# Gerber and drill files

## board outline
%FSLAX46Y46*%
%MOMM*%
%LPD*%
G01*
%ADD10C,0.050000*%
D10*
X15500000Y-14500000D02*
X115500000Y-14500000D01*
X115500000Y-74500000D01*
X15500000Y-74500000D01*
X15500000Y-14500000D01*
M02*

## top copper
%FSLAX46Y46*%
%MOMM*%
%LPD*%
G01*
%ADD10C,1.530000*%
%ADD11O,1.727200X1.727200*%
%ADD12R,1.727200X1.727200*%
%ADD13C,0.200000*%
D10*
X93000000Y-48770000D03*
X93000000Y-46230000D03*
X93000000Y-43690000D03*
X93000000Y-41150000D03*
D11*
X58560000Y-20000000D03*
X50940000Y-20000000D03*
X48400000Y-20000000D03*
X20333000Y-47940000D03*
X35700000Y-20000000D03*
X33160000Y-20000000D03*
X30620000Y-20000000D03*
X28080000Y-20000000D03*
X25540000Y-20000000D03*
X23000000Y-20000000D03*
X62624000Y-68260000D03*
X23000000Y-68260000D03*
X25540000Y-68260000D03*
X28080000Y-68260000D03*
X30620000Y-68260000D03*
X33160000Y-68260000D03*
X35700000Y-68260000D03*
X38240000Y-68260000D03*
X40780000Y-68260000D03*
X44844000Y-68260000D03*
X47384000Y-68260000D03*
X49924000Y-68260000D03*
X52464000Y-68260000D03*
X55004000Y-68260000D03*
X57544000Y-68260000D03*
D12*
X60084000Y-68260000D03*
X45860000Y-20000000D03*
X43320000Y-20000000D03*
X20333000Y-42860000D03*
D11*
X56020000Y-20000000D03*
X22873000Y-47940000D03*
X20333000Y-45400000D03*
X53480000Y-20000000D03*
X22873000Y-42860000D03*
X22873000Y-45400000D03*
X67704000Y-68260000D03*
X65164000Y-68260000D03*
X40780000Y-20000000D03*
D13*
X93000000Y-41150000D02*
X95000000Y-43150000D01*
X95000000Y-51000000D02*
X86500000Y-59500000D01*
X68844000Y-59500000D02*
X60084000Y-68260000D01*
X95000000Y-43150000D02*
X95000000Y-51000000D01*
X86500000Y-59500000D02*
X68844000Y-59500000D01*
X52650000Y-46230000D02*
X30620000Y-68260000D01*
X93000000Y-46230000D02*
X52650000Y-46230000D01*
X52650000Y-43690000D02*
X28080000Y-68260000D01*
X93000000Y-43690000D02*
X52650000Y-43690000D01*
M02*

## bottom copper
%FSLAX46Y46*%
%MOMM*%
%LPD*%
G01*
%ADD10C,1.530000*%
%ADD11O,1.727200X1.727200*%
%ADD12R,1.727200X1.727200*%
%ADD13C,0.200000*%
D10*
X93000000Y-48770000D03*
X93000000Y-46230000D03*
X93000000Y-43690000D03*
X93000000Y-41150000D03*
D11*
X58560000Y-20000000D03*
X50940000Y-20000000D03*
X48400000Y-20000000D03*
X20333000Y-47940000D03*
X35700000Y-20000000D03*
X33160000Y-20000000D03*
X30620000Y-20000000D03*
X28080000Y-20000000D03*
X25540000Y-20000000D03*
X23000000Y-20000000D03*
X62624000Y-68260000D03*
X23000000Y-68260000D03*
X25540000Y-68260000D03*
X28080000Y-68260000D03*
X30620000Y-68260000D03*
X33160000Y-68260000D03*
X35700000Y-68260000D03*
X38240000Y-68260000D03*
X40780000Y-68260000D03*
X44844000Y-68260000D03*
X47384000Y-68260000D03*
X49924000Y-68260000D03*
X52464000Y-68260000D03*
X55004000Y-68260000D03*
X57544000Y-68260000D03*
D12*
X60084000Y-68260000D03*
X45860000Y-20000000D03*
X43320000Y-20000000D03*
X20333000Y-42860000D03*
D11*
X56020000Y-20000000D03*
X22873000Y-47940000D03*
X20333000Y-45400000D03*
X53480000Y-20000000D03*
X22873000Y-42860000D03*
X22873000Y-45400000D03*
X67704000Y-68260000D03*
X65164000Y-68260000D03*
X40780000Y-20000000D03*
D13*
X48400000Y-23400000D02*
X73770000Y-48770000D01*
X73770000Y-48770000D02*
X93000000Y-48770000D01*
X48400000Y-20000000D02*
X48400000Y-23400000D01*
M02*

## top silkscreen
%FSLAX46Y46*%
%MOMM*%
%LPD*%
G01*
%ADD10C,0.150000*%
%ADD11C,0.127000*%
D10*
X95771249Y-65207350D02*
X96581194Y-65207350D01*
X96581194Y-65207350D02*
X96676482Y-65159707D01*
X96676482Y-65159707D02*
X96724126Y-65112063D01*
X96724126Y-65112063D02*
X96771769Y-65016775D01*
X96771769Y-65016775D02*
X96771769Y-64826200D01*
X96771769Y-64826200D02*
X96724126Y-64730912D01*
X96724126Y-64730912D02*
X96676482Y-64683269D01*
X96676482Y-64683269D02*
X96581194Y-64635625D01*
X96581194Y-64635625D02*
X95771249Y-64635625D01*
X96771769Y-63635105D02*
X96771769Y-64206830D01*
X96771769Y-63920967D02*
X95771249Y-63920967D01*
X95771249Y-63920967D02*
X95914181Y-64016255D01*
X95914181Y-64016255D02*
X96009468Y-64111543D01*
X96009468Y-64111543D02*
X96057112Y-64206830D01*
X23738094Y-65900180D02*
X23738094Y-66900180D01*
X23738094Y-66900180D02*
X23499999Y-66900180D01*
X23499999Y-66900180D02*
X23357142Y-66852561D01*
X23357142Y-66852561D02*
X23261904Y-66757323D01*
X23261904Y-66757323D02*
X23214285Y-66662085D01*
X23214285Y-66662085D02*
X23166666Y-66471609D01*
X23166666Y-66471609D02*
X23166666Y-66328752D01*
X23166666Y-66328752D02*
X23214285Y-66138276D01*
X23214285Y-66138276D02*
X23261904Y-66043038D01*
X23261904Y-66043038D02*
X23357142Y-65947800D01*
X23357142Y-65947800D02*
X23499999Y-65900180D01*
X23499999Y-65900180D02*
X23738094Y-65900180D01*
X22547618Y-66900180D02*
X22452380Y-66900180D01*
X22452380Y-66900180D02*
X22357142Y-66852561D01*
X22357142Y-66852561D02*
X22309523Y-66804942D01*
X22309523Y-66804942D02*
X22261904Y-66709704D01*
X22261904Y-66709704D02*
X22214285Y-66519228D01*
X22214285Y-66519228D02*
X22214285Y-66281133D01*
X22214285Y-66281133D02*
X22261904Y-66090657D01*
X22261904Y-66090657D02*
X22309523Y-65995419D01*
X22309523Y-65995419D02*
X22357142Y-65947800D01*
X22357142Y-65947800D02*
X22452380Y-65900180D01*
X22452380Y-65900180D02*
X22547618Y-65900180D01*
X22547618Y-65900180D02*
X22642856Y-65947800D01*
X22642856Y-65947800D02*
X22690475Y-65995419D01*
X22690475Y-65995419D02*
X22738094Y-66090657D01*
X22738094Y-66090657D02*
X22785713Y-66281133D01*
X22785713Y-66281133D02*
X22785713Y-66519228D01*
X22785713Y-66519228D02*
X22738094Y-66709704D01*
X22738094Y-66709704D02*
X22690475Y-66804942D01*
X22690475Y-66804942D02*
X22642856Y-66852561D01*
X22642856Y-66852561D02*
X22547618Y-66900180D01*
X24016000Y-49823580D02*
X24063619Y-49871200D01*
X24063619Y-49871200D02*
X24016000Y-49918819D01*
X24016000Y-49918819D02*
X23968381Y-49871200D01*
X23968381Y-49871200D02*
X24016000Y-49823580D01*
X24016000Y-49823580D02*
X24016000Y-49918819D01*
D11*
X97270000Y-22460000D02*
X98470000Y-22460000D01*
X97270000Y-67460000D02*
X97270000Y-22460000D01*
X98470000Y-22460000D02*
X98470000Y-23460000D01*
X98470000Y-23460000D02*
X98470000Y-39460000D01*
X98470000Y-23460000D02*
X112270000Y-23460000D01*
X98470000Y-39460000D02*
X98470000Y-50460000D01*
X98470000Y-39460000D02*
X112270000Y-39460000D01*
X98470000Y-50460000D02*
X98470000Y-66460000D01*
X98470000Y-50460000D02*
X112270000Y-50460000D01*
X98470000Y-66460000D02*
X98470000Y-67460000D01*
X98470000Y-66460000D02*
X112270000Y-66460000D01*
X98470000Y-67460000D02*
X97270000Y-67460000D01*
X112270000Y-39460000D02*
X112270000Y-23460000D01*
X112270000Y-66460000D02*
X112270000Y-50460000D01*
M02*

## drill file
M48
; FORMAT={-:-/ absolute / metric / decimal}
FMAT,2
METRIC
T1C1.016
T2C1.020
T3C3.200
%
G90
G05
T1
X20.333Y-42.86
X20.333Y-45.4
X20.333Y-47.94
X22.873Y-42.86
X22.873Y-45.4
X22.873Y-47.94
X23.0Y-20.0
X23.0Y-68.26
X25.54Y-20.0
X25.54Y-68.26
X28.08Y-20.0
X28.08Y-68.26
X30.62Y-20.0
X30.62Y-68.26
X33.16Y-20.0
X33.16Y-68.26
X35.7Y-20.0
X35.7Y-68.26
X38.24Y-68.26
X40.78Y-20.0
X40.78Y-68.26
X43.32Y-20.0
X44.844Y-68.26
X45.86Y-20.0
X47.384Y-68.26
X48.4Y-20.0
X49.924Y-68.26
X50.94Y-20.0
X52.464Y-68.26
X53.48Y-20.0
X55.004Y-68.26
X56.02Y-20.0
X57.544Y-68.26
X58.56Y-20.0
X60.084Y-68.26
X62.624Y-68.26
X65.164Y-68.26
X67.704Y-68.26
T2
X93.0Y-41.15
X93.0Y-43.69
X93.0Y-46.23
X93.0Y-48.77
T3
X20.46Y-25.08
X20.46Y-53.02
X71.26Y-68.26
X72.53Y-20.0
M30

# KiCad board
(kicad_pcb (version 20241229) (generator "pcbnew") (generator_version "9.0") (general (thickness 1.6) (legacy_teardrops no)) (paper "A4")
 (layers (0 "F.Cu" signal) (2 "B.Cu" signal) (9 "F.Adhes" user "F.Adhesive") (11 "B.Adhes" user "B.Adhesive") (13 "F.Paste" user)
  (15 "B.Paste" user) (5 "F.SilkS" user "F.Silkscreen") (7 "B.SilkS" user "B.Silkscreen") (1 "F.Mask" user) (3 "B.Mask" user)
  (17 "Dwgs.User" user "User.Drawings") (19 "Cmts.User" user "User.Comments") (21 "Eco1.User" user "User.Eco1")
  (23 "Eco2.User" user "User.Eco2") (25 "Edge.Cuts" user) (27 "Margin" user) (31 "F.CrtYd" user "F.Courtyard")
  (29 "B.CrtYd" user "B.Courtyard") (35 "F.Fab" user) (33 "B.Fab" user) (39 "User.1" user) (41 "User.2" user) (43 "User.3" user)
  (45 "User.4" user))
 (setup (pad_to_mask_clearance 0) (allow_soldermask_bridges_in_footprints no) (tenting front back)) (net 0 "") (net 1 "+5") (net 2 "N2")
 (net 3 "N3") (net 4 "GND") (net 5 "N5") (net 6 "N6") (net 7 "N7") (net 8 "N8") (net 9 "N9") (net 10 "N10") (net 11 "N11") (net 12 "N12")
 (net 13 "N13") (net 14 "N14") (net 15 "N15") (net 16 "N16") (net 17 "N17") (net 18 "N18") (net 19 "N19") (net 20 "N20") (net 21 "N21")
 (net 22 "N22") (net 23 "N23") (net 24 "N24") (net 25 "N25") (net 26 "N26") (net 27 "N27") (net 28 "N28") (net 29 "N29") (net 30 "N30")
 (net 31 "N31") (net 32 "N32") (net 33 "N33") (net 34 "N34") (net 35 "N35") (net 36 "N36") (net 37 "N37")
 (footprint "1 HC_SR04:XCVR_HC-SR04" (layer "F.Cu") (at 93 44.96 90)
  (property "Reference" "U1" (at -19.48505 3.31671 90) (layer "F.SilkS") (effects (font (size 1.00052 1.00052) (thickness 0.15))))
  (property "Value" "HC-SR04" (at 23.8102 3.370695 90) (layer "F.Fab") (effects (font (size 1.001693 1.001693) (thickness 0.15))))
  (fp_line (start 22.5 4.27) (end 22.5 5.47) (stroke (width 0.127) (type solid)) (layer "F.SilkS"))
  (fp_line (start -22.5 4.27) (end 22.5 4.27) (stroke (width 0.127) (type solid)) (layer "F.SilkS"))
  (fp_line (start 22.5 5.47) (end 21.5 5.47) (stroke (width 0.127) (type solid)) (layer "F.SilkS"))
  (fp_line (start 21.5 5.47) (end 5.5 5.47) (stroke (width 0.127) (type solid)) (layer "F.SilkS"))
  (fp_line (start 21.5 5.47) (end 21.5 19.27) (stroke (width 0.127) (type solid)) (layer "F.SilkS"))
  (fp_line (start 5.5 5.47) (end -5.5 5.47) (stroke (width 0.127) (type solid)) (layer "F.SilkS"))
  (fp_line (start 5.5 5.47) (end 5.5 19.27) (stroke (width 0.127) (type solid)) (layer "F.SilkS"))
  (fp_line (start -5.5 5.47) (end -21.5 5.47) (stroke (width 0.127) (type solid)) (layer "F.SilkS"))
  (fp_line (start -5.5 5.47) (end -5.5 19.27) (stroke (width 0.127) (type solid)) (layer "F.SilkS"))
  (fp_line (start -21.5 5.47) (end -22.5 5.47) (stroke (width 0.127) (type solid)) (layer "F.SilkS"))
  (fp_line (start -21.5 5.47) (end -21.5 19.27) (stroke (width 0.127) (type solid)) (layer "F.SilkS"))
  (fp_line (start -22.5 5.47) (end -22.5 4.27) (stroke (width 0.127) (type solid)) (layer "F.SilkS"))
  (fp_line (start 5.5 19.27) (end 21.5 19.27) (stroke (width 0.127) (type solid)) (layer "F.SilkS"))
  (fp_line (start -21.5 19.27) (end -5.5 19.27) (stroke (width 0.127) (type solid)) (layer "F.SilkS"))
  (pad "1" thru_hole circle (at -3.81 0 90) (size 1.53 1.53) (drill 1.02) (layers "*.Cu" "*.Mask") (remove_unused_layers no) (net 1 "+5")
   (solder_mask_margin 0.102))
  (pad "2" thru_hole circle (at -1.27 0 90) (size 1.53 1.53) (drill 1.02) (layers "*.Cu" "*.Mask") (remove_unused_layers no) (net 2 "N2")
   (solder_mask_margin 0.102))
  (pad "3" thru_hole circle (at 1.27 0 90) (size 1.53 1.53) (drill 1.02) (layers "*.Cu" "*.Mask") (remove_unused_layers no) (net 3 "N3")
   (solder_mask_margin 0.102))
  (pad "4" thru_hole circle (at 3.81 0 90) (size 1.53 1.53) (drill 1.02) (layers "*.Cu" "*.Mask") (remove_unused_layers no) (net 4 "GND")
   (solder_mask_margin 0.102)))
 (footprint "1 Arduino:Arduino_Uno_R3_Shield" (layer "F.Cu") (at 86.5 17.46 180)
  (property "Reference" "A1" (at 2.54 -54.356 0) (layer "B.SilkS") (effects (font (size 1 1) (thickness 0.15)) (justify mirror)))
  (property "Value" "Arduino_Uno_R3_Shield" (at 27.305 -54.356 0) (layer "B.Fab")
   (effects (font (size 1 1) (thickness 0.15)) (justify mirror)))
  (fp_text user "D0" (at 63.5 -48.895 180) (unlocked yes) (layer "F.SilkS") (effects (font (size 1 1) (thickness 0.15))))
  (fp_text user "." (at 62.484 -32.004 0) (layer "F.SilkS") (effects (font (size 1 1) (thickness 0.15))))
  (pad "" np_thru_hole circle (at 13.97 -2.54 180) (size 3.2 3.2) (drill 3.2) (layers "*.Cu" "*.Mask"))
  (pad "" np_thru_hole circle (at 15.24 -50.8 180) (size 3.2 3.2) (drill 3.2) (layers "*.Cu" "*.Mask"))
  (pad "" thru_hole oval (at 27.94 -2.54 180) (size 1.7272 1.7272) (drill 1.016) (layers "*.Cu" "*.Mask") (remove_unused_layers no))
  (pad "" np_thru_hole circle (at 66.04 -35.56 180) (size 3.2 3.2) (drill 3.2) (layers "*.Cu" "*.Mask"))
  (pad "" np_thru_hole circle (at 66.04 -7.62 180) (size 3.2 3.2) (drill 3.2) (layers "*.Cu" "*.Mask"))
  (pad "3V3" thru_hole oval (at 35.56 -2.54 180) (size 1.7272 1.7272) (drill 1.016) (layers "*.Cu" "*.Mask") (remove_unused_layers no)
   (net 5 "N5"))
  (pad "5V1" thru_hole oval (at 38.1 -2.54 180) (size 1.7272 1.7272) (drill 1.016) (layers "*.Cu" "*.Mask") (remove_unused_layers no)
   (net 1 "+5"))
  (pad "5V2" thru_hole oval (at 66.167 -30.48 180) (size 1.7272 1.7272) (drill 1.016) (layers "*.Cu" "*.Mask") (remove_unused_layers no)
   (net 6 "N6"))
  (pad "A0" thru_hole oval (at 50.8 -2.54 180) (size 1.7272 1.7272) (drill 1.016) (layers "*.Cu" "*.Mask") (remove_unused_layers no)
   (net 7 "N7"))
  (pad "A1" thru_hole oval (at 53.34 -2.54 180) (size 1.7272 1.7272) (drill 1.016) (layers "*.Cu" "*.Mask") (remove_unused_layers no)
   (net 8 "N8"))
  (pad "A2" thru_hole oval (at 55.88 -2.54 180) (size 1.7272 1.7272) (drill 1.016) (layers "*.Cu" "*.Mask") (remove_unused_layers no)
   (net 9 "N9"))
  (pad "A3" thru_hole oval (at 58.42 -2.54 180) (size 1.7272 1.7272) (drill 1.016) (layers "*.Cu" "*.Mask") (remove_unused_layers no)
   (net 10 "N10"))
  (pad "A4" thru_hole oval (at 60.96 -2.54 180) (size 1.7272 1.7272) (drill 1.016) (layers "*.Cu" "*.Mask") (remove_unused_layers no)
   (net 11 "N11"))
  (pad "A5" thru_hole oval (at 63.5 -2.54 180) (size 1.7272 1.7272) (drill 1.016) (layers "*.Cu" "*.Mask") (remove_unused_layers no)
   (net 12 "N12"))
  (pad "AREF" thru_hole oval (at 23.876 -50.8 180) (size 1.7272 1.7272) (drill 1.016) (layers "*.Cu" "*.Mask") (remove_unused_layers no)
   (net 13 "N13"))
  (pad "D0" thru_hole oval (at 63.5 -50.8 180) (size 1.7272 1.7272) (drill 1.016) (layers "*.Cu" "*.Mask") (remove_unused_layers no)
   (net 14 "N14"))
  (pad "D1" thru_hole oval (at 60.96 -50.8 180) (size 1.7272 1.7272) (drill 1.016) (layers "*.Cu" "*.Mask") (remove_unused_layers no)
   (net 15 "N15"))
  (pad "D2" thru_hole oval (at 58.42 -50.8 180) (size 1.7272 1.7272) (drill 1.016) (layers "*.Cu" "*.Mask") (remove_unused_layers no)
   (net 3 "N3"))
  (pad "D3" thru_hole oval (at 55.88 -50.8 180) (size 1.7272 1.7272) (drill 1.016) (layers "*.Cu" "*.Mask") (remove_unused_layers no)
   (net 2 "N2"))
  (pad "D4" thru_hole oval (at 53.34 -50.8 180) (size 1.7272 1.7272) (drill 1.016) (layers "*.Cu" "*.Mask") (remove_unused_layers no)
   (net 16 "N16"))
  (pad "D5" thru_hole oval (at 50.8 -50.8 180) (size 1.7272 1.7272) (drill 1.016) (layers "*.Cu" "*.Mask") (remove_unused_layers no)
   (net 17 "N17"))
  (pad "D6" thru_hole oval (at 48.26 -50.8 180) (size 1.7272 1.7272) (drill 1.016) (layers "*.Cu" "*.Mask") (remove_unused_layers no)
   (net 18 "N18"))
  (pad "D7" thru_hole oval (at 45.72 -50.8 180) (size 1.7272 1.7272) (drill 1.016) (layers "*.Cu" "*.Mask") (remove_unused_layers no)
   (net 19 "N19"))
  (pad "D8" thru_hole oval (at 41.656 -50.8 180) (size 1.7272 1.7272) (drill 1.016) (layers "*.Cu" "*.Mask") (remove_unused_layers no)
   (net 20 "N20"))
  (pad "D9" thru_hole oval (at 39.116 -50.8 180) (size 1.7272 1.7272) (drill 1.016) (layers "*.Cu" "*.Mask") (remove_unused_layers no)
   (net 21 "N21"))
  (pad "D10" thru_hole oval (at 36.576 -50.8 180) (size 1.7272 1.7272) (drill 1.016) (layers "*.Cu" "*.Mask") (remove_unused_layers no)
   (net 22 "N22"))
  (pad "D11" thru_hole oval (at 34.036 -50.8 180) (size 1.7272 1.7272) (drill 1.016) (layers "*.Cu" "*.Mask") (remove_unused_layers no)
   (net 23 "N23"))
  (pad "D12" thru_hole oval (at 31.496 -50.8 180) (size 1.7272 1.7272) (drill 1.016) (layers "*.Cu" "*.Mask") (remove_unused_layers no)
   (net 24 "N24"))
  (pad "D13" thru_hole oval (at 28.956 -50.8 180) (size 1.7272 1.7272) (drill 1.016) (layers "*.Cu" "*.Mask") (remove_unused_layers no)
   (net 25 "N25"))
  (pad "GND1" thru_hole rect (at 26.416 -50.8 180) (size 1.7272 1.7272) (drill 1.016) (layers "*.Cu" "*.Mask") (remove_unused_layers no)
   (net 4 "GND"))
  (pad "GND2" thru_hole rect (at 40.64 -2.54 180) (size 1.7272 1.7272) (drill 1.016) (layers "*.Cu" "*.Mask") (remove_unused_layers no)
   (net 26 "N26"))
  (pad "GND3" thru_hole rect (at 43.18 -2.54 180) (size 1.7272 1.7272) (drill 1.016) (layers "*.Cu" "*.Mask") (remove_unused_layers no)
   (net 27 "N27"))
  (pad "GND4" thru_hole rect (at 66.167 -25.4 180) (size 1.7272 1.7272) (drill 1.016) (layers "*.Cu" "*.Mask") (remove_unused_layers no)
   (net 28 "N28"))
  (pad "IORF" thru_hole oval (at 30.48 -2.54 180) (size 1.7272 1.7272) (drill 1.016) (layers "*.Cu" "*.Mask") (remove_unused_layers no)
   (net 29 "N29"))
  (pad "MISO" thru_hole oval (at 63.627 -30.48 180) (size 1.7272 1.7272) (drill 1.016) (layers "*.Cu" "*.Mask") (remove_unused_layers no)
   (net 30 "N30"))
  (pad "MOSI" thru_hole oval (at 66.167 -27.94 180) (size 1.7272 1.7272) (drill 1.016) (layers "*.Cu" "*.Mask") (remove_unused_layers no)
   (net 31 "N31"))
  (pad "RST1" thru_hole oval (at 33.02 -2.54 180) (size 1.7272 1.7272) (drill 1.016) (layers "*.Cu" "*.Mask") (remove_unused_layers no)
   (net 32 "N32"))
  (pad "RST2" thru_hole oval (at 63.627 -25.4 180) (size 1.7272 1.7272) (drill 1.016) (layers "*.Cu" "*.Mask") (remove_unused_layers no)
   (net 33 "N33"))
  (pad "SCK" thru_hole oval (at 63.627 -27.94 180) (size 1.7272 1.7272) (drill 1.016) (layers "*.Cu" "*.Mask") (remove_unused_layers no)
   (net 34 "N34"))
  (pad "SCL" thru_hole oval (at 18.796 -50.8 180) (size 1.7272 1.7272) (drill 1.016) (layers "*.Cu" "*.Mask") (remove_unused_layers no)
   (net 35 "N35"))
  (pad "SDA" thru_hole oval (at 21.336 -50.8 180) (size 1.7272 1.7272) (drill 1.016) (layers "*.Cu" "*.Mask") (remove_unused_layers no)
   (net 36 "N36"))
  (pad "VIN" thru_hole oval (at 45.72 -2.54 180) (size 1.7272 1.7272) (drill 1.016) (layers "*.Cu" "*.Mask") (remove_unused_layers no)
   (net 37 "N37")))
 (gr_rect (start 15.5 14.5) (end 115.5 74.5) (stroke (width 0.05) (type default)) (fill no) (layer "Edge.Cuts"))
 (segment (start 93 41.15) (end 95 43.15) (width 0.2) (layer "F.Cu") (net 4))
 (segment (start 95 51) (end 86.5 59.5) (width 0.2) (layer "F.Cu") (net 4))
 (segment (start 68.844 59.5) (end 60.084 68.26) (width 0.2) (layer "F.Cu") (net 4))
 (segment (start 95 43.15) (end 95 51) (width 0.2) (layer "F.Cu") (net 4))
 (segment (start 86.5 59.5) (end 68.844 59.5) (width 0.2) (layer "F.Cu") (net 4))
 (segment (start 52.65 46.23) (end 30.62 68.26) (width 0.2) (layer "F.Cu") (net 2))
 (segment (start 93 46.23) (end 52.65 46.23) (width 0.2) (layer "F.Cu") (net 2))
 (segment (start 52.65 43.69) (end 28.08 68.26) (width 0.2) (layer "F.Cu") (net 3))
 (segment (start 93 43.69) (end 52.65 43.69) (width 0.2) (layer "F.Cu") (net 3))
 (segment (start 48.4 23.4) (end 73.77 48.77) (width 0.2) (layer "B.Cu") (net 1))
 (segment (start 73.77 48.77) (end 93 48.77) (width 0.2) (layer "B.Cu") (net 1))
 (segment (start 48.4 20) (end 48.4 23.4) (width 0.2) (layer "B.Cu") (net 1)))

